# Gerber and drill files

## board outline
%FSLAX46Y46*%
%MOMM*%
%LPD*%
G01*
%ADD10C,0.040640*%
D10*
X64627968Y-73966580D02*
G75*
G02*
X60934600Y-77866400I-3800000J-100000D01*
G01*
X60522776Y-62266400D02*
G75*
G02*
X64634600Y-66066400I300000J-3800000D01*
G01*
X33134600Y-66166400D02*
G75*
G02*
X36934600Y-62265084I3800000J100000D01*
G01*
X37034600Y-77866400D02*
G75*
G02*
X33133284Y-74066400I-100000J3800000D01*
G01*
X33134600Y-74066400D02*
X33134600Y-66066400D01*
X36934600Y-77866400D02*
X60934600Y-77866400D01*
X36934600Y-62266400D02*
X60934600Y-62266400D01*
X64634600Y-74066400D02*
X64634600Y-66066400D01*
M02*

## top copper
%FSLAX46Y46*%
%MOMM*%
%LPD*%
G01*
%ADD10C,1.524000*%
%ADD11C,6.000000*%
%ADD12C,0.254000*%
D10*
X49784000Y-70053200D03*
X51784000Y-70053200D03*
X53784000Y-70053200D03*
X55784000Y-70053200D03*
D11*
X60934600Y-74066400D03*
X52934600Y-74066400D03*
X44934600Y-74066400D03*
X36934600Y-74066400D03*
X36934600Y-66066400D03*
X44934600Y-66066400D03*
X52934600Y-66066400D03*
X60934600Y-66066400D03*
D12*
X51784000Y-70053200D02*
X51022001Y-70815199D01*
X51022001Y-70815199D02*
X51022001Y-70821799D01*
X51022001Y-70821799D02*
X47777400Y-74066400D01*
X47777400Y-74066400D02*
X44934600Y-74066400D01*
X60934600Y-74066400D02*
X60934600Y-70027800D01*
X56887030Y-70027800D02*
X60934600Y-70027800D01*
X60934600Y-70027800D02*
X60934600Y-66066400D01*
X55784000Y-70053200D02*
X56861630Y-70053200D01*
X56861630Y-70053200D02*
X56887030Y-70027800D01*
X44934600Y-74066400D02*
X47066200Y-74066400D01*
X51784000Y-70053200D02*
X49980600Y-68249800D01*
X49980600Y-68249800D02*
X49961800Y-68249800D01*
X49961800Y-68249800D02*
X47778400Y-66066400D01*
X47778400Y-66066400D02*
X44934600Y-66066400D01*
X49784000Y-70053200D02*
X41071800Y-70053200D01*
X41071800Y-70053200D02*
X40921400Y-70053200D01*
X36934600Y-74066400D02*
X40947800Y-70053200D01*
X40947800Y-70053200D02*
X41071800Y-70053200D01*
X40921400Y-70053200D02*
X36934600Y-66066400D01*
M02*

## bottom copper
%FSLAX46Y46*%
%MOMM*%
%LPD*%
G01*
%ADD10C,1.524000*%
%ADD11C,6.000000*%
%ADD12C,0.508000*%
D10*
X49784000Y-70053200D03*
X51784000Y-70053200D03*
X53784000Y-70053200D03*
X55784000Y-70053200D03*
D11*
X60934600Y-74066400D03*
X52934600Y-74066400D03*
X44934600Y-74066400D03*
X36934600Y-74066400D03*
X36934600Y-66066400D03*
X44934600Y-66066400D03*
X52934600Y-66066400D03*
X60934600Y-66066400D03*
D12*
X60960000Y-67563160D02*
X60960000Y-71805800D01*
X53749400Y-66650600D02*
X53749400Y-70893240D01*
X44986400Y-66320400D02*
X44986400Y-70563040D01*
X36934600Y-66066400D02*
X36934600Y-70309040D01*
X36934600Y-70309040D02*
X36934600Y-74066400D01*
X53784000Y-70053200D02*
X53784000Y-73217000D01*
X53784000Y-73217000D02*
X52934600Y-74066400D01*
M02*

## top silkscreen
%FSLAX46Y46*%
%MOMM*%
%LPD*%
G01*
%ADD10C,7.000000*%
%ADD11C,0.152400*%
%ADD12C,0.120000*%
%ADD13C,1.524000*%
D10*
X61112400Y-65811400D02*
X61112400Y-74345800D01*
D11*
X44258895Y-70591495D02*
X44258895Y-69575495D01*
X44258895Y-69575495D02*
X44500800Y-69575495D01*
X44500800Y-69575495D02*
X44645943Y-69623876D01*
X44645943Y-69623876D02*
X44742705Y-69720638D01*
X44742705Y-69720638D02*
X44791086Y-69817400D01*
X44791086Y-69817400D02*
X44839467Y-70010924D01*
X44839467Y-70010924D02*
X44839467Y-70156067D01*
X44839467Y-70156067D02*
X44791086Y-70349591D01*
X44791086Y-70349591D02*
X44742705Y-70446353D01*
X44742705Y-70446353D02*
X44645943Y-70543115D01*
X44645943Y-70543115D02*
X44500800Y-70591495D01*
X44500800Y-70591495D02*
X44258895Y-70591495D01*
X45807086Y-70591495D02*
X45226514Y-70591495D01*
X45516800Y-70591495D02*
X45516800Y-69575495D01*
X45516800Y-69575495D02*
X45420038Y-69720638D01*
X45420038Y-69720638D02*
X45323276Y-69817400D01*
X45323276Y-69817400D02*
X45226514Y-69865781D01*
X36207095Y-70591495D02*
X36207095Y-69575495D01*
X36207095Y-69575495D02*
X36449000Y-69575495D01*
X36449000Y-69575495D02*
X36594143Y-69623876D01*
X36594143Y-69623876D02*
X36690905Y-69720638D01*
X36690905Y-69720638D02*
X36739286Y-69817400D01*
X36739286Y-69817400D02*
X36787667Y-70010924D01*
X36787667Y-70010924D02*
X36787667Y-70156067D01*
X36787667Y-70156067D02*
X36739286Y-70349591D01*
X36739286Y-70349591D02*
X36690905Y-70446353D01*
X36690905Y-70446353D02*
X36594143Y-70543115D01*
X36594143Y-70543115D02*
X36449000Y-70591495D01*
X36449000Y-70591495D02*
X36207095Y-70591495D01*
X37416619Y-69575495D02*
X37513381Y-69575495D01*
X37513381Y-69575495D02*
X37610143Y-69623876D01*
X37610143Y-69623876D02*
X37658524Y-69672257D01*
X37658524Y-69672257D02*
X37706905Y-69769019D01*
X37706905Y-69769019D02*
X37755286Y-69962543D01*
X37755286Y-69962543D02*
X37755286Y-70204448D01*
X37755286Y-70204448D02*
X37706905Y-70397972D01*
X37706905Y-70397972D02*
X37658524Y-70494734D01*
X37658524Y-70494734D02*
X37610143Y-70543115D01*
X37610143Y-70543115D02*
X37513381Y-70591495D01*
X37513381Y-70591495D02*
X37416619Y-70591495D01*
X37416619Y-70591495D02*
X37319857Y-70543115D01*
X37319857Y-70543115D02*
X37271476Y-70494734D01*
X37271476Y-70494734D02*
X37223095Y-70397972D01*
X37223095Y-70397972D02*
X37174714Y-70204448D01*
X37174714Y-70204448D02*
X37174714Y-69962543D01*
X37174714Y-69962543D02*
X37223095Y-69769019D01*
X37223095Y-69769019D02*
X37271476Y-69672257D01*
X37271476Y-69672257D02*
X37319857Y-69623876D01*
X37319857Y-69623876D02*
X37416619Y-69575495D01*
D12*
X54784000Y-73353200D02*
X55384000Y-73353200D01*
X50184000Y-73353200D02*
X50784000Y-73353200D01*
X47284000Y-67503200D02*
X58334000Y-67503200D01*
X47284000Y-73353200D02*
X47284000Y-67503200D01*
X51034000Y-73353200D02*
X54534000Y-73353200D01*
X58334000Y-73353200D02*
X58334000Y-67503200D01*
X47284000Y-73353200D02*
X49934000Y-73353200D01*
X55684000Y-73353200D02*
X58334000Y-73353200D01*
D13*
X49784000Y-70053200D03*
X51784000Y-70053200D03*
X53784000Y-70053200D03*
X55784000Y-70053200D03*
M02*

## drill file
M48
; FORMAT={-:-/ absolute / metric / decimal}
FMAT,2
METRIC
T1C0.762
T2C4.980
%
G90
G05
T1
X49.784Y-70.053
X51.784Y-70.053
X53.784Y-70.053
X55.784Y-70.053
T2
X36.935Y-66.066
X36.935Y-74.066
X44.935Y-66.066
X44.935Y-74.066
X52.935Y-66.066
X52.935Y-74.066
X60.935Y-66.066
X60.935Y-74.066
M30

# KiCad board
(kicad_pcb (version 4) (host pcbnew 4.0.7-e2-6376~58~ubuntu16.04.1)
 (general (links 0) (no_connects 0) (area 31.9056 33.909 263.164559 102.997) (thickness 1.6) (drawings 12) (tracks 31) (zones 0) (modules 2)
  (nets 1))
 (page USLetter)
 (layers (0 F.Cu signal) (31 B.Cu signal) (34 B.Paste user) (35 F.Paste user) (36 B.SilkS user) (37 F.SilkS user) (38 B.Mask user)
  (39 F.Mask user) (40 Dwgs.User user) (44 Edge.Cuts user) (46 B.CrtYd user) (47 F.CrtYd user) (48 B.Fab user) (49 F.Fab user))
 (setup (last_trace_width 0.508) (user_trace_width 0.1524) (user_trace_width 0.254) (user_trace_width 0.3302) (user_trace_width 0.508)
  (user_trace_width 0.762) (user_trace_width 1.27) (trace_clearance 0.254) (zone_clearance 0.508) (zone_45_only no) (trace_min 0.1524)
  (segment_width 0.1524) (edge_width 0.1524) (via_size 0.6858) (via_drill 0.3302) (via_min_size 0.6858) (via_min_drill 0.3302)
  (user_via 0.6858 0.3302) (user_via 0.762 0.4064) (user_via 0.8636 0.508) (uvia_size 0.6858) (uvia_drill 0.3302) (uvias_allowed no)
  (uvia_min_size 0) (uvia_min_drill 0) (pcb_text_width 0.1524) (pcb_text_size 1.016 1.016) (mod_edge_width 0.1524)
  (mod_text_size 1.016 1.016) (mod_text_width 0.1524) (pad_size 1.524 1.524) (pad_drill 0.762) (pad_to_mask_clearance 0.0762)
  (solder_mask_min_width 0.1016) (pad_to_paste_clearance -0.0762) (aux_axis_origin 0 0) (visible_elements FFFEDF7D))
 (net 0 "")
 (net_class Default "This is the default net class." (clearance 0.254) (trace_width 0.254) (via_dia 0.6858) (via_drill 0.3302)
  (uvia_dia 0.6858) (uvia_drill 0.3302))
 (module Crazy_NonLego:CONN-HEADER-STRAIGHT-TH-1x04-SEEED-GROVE (layer F.Cu) (at 49.784 70.0532 90)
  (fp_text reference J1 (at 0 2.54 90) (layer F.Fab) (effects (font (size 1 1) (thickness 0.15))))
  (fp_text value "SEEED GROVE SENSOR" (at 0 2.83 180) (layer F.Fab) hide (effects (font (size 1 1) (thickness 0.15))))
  (fp_line (start -3.3 5) (end -3.3 5.6) (layer F.SilkS) (width 0.12))
  (fp_line (start -3.3 0.4) (end -3.3 1) (layer F.SilkS) (width 0.12))
  (fp_line (start 2.55 -2.5) (end 2.55 8.55) (layer F.SilkS) (width 0.12))
  (fp_line (start -3.3 -2.5) (end 2.55 -2.5) (layer F.SilkS) (width 0.12))
  (fp_line (start -3.3 1.25) (end -3.3 4.75) (layer F.SilkS) (width 0.12))
  (fp_line (start -3.3 8.55) (end 2.55 8.55) (layer F.SilkS) (width 0.12))
  (fp_line (start -3.3 -2.5) (end -3.3 0.15) (layer F.SilkS) (width 0.12))
  (fp_line (start -3.3 5.9) (end -3.3 8.55) (layer F.SilkS) (width 0.12))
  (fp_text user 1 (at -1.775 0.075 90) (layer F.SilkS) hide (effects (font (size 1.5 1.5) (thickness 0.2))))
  (pad 1 thru_hole circle (at 0 0 90) (size 1.524 1.524) (drill 0.762) (layers *.Cu *.Mask F.SilkS))
  (pad 2 thru_hole circle (at 0 2 90) (size 1.524 1.524) (drill 0.762) (layers *.Cu *.Mask F.SilkS))
  (pad 3 thru_hole circle (at 0 4 90) (size 1.524 1.524) (drill 0.762) (layers *.Cu *.Mask F.SilkS))
  (pad 4 thru_hole circle (at 0 6 90) (size 1.524 1.524) (drill 0.762) (layers *.Cu *.Mask F.SilkS)))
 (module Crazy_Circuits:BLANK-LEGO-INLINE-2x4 (layer F.Cu) (at 60.9346 74.0664 90)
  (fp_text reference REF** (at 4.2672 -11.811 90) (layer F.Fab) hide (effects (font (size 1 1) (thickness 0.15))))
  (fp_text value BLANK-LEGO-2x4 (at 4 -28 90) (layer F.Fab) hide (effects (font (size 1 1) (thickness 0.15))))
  (fp_arc (start -0.00018 -0.106632) (end 0.09982 3.693368) (angle 89.9) (layer Edge.Cuts) (width 0.04064))
  (fp_arc (start 8 -0.111824) (end 11.8 -0.411824) (angle 94.51398846) (layer Edge.Cuts) (width 0.04064))
  (fp_arc (start 8 -24) (end 7.9 -27.8) (angle 91.50743576) (layer Edge.Cuts) (width 0.04064))
  (fp_arc (start 0 -24) (end -3.8 -23.9) (angle 91.50743576) (layer Edge.Cuts) (width 0.04064))
  (fp_line (start 0 -27.8) (end 8 -27.8) (layer Edge.Cuts) (width 0.04064))
  (fp_line (start -3.8 -24) (end -3.8 0) (layer Edge.Cuts) (width 0.04064))
  (fp_line (start 11.8 -24) (end 11.8 0) (layer Edge.Cuts) (width 0.04064))
  (fp_line (start 0 3.7) (end 8 3.7) (layer Edge.Cuts) (width 0.04064))
  (pad 4 thru_hole circle (at 0 0 90) (size 6 6) (drill 4.98) (layers *.Cu *.Mask))
  (pad 3 thru_hole circle (at 0 -8 90) (size 6 6) (drill 4.98) (layers *.Cu))
  (pad 2 thru_hole circle (at 0 -16 90) (size 6 6) (drill 4.98) (layers *.Cu *.Mask))
  (pad 1 thru_hole circle (at 0 -24 90) (size 6 6) (drill 4.98) (layers *.Cu *.Mask))
  (pad 1 thru_hole circle (at 8 -24 90) (size 6 6) (drill 4.98) (layers *.Cu *.Mask))
  (pad 2 thru_hole circle (at 8 -16 90) (size 6 6) (drill 4.98) (layers *.Cu *.Mask))
  (pad 3 thru_hole circle (at 8 -8 90) (size 6 6) (drill 4.98) (layers *.Cu))
  (pad 4 thru_hole circle (at 8 0 90) (size 6 6) (drill 4.98) (layers *.Cu *.Mask)))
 (gr_line (start 61.1124 65.8114) (end 61.1124 74.3458) (layer F.SilkS) (width 7))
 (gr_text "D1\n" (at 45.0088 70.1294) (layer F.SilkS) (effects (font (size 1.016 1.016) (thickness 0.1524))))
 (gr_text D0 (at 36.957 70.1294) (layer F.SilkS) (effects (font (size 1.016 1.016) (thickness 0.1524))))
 (segment (start 60.96 67.56316) (end 60.96 71.8058) (width 0.508) (layer B.Cu) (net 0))
 (segment (start 53.7494 66.6506) (end 53.7494 70.89324) (width 0.508) (layer B.Cu) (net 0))
 (segment (start 44.9864 66.3204) (end 44.9864 70.56304) (width 0.508) (layer B.Cu) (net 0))
 (segment (start 36.9346 66.0664) (end 36.9346 70.30904) (width 0.508) (layer B.Cu) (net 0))
 (segment (start 36.9346 70.30904) (end 36.9346 74.0664) (width 0.508) (layer B.Cu) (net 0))
 (segment (start 60.9346 70.30904) (end 60.9346 74.0664) (width 0.508) (layer B.Mask) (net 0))
 (segment (start 53.784 70.0532) (end 53.784 73.217) (width 0.508) (layer B.Cu) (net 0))
 (segment (start 53.784 73.217) (end 52.9346 74.0664) (width 0.508) (layer B.Cu) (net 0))
 (segment (start 53.784 70.0532) (end 53.784 66.9158) (width 0.508) (layer B.Mask) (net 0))
 (segment (start 53.784 66.9158) (end 52.9346 66.0664) (width 0.508) (layer B.Mask) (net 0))
 (segment (start 44.9346 70.30904) (end 44.9346 74.0664) (width 0.508) (layer B.Mask) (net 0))
 (segment (start 36.9346 70.30904) (end 36.9346 74.0664) (width 0.508) (layer B.Mask) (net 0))
 (segment (start 51.784 70.0532) (end 51.022001 70.815199) (width 0.254) (layer F.Cu) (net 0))
 (segment (start 51.022001 70.815199) (end 51.022001 70.821799) (width 0.254) (layer F.Cu) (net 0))
 (segment (start 51.022001 70.821799) (end 47.7774 74.0664) (width 0.254) (layer F.Cu) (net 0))
 (segment (start 47.7774 74.0664) (end 44.9346 74.0664) (width 0.254) (layer F.Cu) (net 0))
 (segment (start 60.9346 74.0664) (end 60.9346 70.0278) (width 0.254) (layer F.Cu) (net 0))
 (segment (start 56.88703 70.0278) (end 60.9346 70.0278) (width 0.254) (layer F.Cu) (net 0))
 (segment (start 60.9346 70.0278) (end 60.9346 66.0664) (width 0.254) (layer F.Cu) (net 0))
 (segment (start 55.784 70.0532) (end 56.86163 70.0532) (width 0.254) (layer F.Cu) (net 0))
 (segment (start 56.86163 70.0532) (end 56.88703 70.0278) (width 0.254) (layer F.Cu) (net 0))
 (segment (start 44.9346 74.0664) (end 47.0662 74.0664) (width 0.254) (layer F.Cu) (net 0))
 (segment (start 51.784 70.0532) (end 49.9806 68.2498) (width 0.254) (layer F.Cu) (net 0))
 (segment (start 49.9806 68.2498) (end 49.9618 68.2498) (width 0.254) (layer F.Cu) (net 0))
 (segment (start 49.9618 68.2498) (end 47.7784 66.0664) (width 0.254) (layer F.Cu) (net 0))
 (segment (start 47.7784 66.0664) (end 44.9346 66.0664) (width 0.254) (layer F.Cu) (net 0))
 (segment (start 49.784 70.0532) (end 41.0718 70.0532) (width 0.254) (layer F.Cu) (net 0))
 (segment (start 41.0718 70.0532) (end 40.9214 70.0532) (width 0.254) (layer F.Cu) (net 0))
 (segment (start 36.9346 74.0664) (end 40.9478 70.0532) (width 0.254) (layer F.Cu) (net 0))
 (segment (start 40.9478 70.0532) (end 41.0718 70.0532) (width 0.254) (layer F.Cu) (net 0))
 (segment (start 40.9214 70.0532) (end 36.9346 66.0664) (width 0.254) (layer F.Cu) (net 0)))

